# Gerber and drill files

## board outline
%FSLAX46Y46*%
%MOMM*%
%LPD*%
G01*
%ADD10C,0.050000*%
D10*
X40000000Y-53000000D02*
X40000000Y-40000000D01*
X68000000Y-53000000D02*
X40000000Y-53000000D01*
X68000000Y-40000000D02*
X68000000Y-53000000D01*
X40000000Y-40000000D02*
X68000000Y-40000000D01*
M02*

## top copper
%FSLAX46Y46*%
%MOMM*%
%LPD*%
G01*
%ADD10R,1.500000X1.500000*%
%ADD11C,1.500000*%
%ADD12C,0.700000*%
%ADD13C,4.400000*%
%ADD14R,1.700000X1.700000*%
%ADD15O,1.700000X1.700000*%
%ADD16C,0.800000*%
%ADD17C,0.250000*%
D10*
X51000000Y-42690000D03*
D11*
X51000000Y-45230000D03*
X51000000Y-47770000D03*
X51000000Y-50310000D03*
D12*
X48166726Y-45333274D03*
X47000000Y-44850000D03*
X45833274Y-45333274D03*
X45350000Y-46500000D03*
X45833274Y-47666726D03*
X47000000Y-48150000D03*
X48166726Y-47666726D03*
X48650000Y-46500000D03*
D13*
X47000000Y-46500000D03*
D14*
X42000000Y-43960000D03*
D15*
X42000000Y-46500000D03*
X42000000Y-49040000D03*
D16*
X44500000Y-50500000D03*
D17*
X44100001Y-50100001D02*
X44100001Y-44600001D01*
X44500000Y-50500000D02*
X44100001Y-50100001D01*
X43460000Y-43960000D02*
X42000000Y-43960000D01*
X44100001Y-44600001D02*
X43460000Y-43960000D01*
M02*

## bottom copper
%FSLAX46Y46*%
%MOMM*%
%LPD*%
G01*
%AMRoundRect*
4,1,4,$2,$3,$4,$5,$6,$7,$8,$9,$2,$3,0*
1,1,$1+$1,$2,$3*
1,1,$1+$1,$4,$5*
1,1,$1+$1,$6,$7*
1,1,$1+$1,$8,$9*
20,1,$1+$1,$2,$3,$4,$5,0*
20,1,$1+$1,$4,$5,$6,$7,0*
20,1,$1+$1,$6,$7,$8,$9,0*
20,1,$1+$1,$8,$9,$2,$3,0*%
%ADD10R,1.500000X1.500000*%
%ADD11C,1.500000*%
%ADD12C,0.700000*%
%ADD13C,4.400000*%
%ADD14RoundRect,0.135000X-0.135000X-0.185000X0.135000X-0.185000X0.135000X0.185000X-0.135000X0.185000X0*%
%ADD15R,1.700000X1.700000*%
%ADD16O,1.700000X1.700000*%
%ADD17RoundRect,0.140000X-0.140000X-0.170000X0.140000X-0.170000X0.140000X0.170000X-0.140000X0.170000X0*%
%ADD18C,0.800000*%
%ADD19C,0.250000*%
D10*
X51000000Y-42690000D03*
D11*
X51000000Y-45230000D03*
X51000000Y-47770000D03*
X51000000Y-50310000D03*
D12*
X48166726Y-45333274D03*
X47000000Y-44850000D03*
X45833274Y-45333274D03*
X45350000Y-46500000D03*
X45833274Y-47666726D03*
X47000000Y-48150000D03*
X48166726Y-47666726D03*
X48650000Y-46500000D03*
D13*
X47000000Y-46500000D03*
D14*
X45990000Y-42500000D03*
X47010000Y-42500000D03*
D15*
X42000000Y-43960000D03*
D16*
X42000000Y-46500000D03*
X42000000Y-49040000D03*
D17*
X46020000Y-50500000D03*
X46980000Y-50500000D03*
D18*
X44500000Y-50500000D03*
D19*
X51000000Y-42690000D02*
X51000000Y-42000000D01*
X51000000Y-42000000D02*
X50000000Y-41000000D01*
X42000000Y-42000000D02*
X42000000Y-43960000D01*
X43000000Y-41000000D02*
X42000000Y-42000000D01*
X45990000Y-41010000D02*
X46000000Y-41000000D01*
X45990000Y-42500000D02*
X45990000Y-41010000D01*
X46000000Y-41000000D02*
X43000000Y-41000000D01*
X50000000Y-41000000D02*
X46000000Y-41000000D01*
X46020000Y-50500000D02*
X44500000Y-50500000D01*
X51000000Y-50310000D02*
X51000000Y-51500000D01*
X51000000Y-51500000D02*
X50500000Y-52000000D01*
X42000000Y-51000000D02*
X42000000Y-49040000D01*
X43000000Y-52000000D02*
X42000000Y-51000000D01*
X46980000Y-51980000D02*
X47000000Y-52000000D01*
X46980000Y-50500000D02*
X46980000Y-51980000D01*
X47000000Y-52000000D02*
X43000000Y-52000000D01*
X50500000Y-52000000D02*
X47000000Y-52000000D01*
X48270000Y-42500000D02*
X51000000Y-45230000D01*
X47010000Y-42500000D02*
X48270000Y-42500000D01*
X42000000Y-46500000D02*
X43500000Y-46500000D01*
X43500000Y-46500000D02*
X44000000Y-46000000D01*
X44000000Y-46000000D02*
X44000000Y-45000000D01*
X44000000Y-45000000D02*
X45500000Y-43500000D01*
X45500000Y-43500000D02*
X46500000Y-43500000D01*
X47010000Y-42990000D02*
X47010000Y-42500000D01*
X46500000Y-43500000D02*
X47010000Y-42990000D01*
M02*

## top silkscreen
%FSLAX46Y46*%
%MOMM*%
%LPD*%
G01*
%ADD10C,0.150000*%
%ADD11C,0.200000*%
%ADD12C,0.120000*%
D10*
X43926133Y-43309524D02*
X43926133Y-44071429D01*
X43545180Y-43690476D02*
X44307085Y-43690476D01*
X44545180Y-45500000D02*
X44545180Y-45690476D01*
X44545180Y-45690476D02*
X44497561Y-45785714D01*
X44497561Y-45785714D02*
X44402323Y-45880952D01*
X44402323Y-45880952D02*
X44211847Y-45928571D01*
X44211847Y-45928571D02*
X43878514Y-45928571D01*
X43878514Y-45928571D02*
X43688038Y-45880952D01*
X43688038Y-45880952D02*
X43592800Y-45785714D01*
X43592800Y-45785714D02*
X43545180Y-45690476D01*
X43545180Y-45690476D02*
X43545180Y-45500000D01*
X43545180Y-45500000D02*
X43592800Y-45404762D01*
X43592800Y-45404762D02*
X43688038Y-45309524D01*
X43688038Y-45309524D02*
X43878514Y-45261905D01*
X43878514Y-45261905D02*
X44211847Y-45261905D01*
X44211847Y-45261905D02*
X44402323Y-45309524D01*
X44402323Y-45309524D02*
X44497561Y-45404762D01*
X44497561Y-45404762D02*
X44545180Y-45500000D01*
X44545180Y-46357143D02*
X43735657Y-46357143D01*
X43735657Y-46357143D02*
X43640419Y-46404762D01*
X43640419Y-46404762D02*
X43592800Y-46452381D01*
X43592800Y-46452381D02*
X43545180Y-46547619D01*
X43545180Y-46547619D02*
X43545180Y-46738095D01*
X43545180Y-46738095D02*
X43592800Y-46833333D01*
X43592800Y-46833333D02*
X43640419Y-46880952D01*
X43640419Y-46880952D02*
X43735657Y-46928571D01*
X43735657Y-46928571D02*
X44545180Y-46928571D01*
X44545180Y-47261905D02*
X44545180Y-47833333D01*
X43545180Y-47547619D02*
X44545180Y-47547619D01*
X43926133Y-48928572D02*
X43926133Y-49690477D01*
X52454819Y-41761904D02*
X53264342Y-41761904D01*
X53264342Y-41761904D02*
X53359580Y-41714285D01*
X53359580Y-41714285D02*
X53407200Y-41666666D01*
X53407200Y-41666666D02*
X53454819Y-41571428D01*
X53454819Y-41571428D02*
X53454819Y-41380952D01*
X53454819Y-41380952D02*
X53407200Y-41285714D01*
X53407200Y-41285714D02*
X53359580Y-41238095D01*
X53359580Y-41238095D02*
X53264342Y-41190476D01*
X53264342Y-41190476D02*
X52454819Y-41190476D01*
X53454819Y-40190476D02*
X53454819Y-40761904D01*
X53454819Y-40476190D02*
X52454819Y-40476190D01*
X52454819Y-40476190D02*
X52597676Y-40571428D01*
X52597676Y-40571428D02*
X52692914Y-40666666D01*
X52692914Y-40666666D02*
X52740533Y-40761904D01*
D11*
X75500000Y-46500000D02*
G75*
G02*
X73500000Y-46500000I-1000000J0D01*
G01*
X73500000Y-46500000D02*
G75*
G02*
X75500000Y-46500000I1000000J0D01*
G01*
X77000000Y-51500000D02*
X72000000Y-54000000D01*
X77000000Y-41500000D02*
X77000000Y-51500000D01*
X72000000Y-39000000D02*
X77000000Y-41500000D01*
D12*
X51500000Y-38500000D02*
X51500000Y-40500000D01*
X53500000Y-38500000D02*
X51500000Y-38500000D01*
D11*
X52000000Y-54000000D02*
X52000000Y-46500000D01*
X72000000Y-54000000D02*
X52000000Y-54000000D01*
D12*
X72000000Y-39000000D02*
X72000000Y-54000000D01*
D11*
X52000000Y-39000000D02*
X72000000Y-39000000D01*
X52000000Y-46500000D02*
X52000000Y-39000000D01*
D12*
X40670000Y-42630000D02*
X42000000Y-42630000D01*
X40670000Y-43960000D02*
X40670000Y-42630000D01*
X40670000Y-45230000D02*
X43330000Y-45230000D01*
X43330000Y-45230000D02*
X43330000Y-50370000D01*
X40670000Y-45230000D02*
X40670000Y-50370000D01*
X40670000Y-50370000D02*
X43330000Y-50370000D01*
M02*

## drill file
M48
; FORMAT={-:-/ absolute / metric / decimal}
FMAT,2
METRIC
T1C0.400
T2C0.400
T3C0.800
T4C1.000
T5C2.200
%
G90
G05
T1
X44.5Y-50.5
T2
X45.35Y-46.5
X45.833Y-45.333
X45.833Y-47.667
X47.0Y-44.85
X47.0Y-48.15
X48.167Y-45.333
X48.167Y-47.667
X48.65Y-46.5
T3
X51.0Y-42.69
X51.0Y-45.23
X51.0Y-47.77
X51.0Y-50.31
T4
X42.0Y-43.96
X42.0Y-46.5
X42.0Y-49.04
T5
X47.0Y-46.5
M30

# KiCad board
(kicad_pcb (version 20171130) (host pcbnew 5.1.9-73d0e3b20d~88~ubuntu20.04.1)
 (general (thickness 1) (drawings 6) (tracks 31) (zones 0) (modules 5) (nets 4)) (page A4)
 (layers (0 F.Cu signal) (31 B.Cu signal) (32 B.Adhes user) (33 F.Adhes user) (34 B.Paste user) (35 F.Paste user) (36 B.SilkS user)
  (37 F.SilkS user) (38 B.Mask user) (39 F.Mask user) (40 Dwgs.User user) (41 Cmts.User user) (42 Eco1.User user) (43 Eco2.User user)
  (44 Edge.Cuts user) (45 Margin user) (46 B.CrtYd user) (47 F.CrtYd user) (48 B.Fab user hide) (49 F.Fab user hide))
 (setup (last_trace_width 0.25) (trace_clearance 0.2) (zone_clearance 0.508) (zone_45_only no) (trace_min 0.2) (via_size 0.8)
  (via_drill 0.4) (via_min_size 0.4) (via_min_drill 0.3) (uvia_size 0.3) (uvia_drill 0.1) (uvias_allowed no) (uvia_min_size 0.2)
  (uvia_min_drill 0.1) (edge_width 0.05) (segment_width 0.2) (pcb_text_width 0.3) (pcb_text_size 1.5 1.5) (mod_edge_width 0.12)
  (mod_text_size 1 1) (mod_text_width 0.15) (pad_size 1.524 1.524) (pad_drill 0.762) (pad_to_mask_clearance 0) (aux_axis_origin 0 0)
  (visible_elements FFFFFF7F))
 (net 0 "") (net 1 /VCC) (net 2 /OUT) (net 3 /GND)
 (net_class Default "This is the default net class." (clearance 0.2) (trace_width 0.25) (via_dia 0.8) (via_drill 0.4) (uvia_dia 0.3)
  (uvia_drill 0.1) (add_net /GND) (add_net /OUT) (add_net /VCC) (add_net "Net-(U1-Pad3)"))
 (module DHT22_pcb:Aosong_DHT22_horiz (layer F.Cu) (at 51 46.5)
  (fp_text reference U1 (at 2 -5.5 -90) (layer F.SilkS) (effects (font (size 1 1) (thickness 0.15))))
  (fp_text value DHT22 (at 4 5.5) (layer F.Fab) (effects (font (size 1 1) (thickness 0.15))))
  (fp_circle (center 23.5 0) (end 24.5 0) (layer F.SilkS) (width 0.2))
  (fp_line (start 26 5) (end 21 7.5) (layer F.SilkS) (width 0.2))
  (fp_line (start 26 -5) (end 26 5) (layer F.SilkS) (width 0.2))
  (fp_line (start 21 -7.5) (end 26 -5) (layer F.SilkS) (width 0.2))
  (fp_line (start 0.5 -8) (end 0.5 -6) (layer F.SilkS) (width 0.12))
  (fp_line (start 2.5 -8) (end 0.5 -8) (layer F.SilkS) (width 0.12))
  (fp_line (start 1 7.5) (end 1 0) (layer F.SilkS) (width 0.2))
  (fp_line (start 21 7.5) (end 1 7.5) (layer F.SilkS) (width 0.2))
  (fp_line (start 21 -7.5) (end 21 7.5) (layer F.SilkS) (width 0.12))
  (fp_line (start 1 -7.5) (end 21 -7.5) (layer F.SilkS) (width 0.2))
  (fp_line (start 1 0) (end 1 -7.5) (layer F.SilkS) (width 0.2))
  (pad 1 thru_hole rect (at 0 -3.81) (size 1.5 1.5) (drill 0.8) (layers *.Cu *.Mask) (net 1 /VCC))
  (pad 2 thru_hole circle (at 0 -1.27) (size 1.5 1.5) (drill 0.8) (layers *.Cu *.Mask) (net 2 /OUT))
  (pad 3 thru_hole circle (at 0 1.27) (size 1.5 1.5) (drill 0.8) (layers *.Cu *.Mask))
  (pad 4 thru_hole circle (at 0 3.81) (size 1.5 1.5) (drill 0.8) (layers *.Cu *.Mask) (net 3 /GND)))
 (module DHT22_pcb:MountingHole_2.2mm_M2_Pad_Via (layer F.Cu) (at 47 46.5)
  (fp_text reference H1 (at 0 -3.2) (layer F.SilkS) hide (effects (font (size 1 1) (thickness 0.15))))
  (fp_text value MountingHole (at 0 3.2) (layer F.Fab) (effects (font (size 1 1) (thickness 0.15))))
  (pad 1 thru_hole circle (at 1.166726 -1.166726) (size 0.7 0.7) (drill 0.4) (layers *.Cu *.Mask))
  (pad 1 thru_hole circle (at 0 -1.65) (size 0.7 0.7) (drill 0.4) (layers *.Cu *.Mask))
  (pad 1 thru_hole circle (at -1.166726 -1.166726) (size 0.7 0.7) (drill 0.4) (layers *.Cu *.Mask))
  (pad 1 thru_hole circle (at -1.65 0) (size 0.7 0.7) (drill 0.4) (layers *.Cu *.Mask))
  (pad 1 thru_hole circle (at -1.166726 1.166726) (size 0.7 0.7) (drill 0.4) (layers *.Cu *.Mask))
  (pad 1 thru_hole circle (at 0 1.65) (size 0.7 0.7) (drill 0.4) (layers *.Cu *.Mask))
  (pad 1 thru_hole circle (at 1.166726 1.166726) (size 0.7 0.7) (drill 0.4) (layers *.Cu *.Mask))
  (pad 1 thru_hole circle (at 1.65 0) (size 0.7 0.7) (drill 0.4) (layers *.Cu *.Mask))
  (pad 1 thru_hole circle (at 0 0) (size 4.4 4.4) (drill 2.2) (layers *.Cu *.Mask)))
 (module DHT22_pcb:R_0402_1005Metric (layer B.Cu) (at 46.5 42.5)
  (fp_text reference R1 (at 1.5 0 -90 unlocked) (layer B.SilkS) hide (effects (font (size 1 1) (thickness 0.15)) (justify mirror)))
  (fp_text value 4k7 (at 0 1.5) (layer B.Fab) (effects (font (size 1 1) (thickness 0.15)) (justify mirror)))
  (pad 1 smd roundrect (at -0.51 0) (size 0.54 0.64) (layers B.Cu B.Paste B.Mask) (roundrect_rratio 0.25) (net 1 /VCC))
  (pad 2 smd roundrect (at 0.51 0) (size 0.54 0.64) (layers B.Cu B.Paste B.Mask) (roundrect_rratio 0.25) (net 2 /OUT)))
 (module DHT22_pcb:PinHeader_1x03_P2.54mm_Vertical (layer F.Cu) (at 42 43.96)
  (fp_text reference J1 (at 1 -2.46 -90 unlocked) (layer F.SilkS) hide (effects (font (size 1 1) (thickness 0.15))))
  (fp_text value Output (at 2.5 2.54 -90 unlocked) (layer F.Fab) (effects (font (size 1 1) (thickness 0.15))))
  (fp_line (start -1.33 -1.33) (end 0 -1.33) (layer F.SilkS) (width 0.12))
  (fp_line (start -1.33 0) (end -1.33 -1.33) (layer F.SilkS) (width 0.12))
  (fp_line (start -1.33 1.27) (end 1.33 1.27) (layer F.SilkS) (width 0.12))
  (fp_line (start 1.33 1.27) (end 1.33 6.41) (layer F.SilkS) (width 0.12))
  (fp_line (start -1.33 1.27) (end -1.33 6.41) (layer F.SilkS) (width 0.12))
  (fp_line (start -1.33 6.41) (end 1.33 6.41) (layer F.SilkS) (width 0.12))
  (pad 1 thru_hole rect (at 0 0) (size 1.7 1.7) (drill 1) (layers *.Cu *.Mask) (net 1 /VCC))
  (pad 2 thru_hole oval (at 0 2.54) (size 1.7 1.7) (drill 1) (layers *.Cu *.Mask) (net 2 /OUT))
  (pad 3 thru_hole oval (at 0 5.08) (size 1.7 1.7) (drill 1) (layers *.Cu *.Mask) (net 3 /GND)))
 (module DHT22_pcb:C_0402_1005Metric (layer B.Cu) (at 46.5 50.5)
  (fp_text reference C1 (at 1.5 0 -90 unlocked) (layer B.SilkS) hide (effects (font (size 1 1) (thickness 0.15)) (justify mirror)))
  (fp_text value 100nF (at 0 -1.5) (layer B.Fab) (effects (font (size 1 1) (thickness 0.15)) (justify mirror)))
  (pad 1 smd roundrect (at -0.48 0) (size 0.56 0.62) (layers B.Cu B.Paste B.Mask) (roundrect_rratio 0.25) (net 1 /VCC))
  (pad 2 smd roundrect (at 0.48 0) (size 0.56 0.62) (layers B.Cu B.Paste B.Mask) (roundrect_rratio 0.25) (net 3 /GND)))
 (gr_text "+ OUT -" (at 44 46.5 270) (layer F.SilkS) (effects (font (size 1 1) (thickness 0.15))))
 (gr_line (start 40 53) (end 40 40) (layer Edge.Cuts) (width 0.05))
 (gr_line (start 68 53) (end 40 53) (layer Edge.Cuts) (width 0.05))
 (gr_line (start 68 40) (end 68 53) (layer Edge.Cuts) (width 0.05))
 (gr_line (start 40 40) (end 68 40) (layer Edge.Cuts) (width 0.05))
 (segment (start 51 42.69) (end 51 42) (width 0.25) (layer B.Cu) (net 1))
 (segment (start 51 42) (end 50 41) (width 0.25) (layer B.Cu) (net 1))
 (segment (start 42 42) (end 42 43.96) (width 0.25) (layer B.Cu) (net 1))
 (segment (start 43 41) (end 42 42) (width 0.25) (layer B.Cu) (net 1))
 (segment (start 45.99 41.01) (end 46 41) (width 0.25) (layer B.Cu) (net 1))
 (segment (start 45.99 42.5) (end 45.99 41.01) (width 0.25) (layer B.Cu) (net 1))
 (segment (start 46 41) (end 43 41) (width 0.25) (layer B.Cu) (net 1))
 (segment (start 50 41) (end 46 41) (width 0.25) (layer B.Cu) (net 1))
 (via (at 44.5 50.5) (size 0.8) (drill 0.4) (layers F.Cu B.Cu) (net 1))
 (segment (start 46.02 50.5) (end 44.5 50.5) (width 0.25) (layer B.Cu) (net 1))
 (segment (start 44.100001 50.100001) (end 44.100001 44.600001) (width 0.25) (layer F.Cu) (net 1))
 (segment (start 44.5 50.5) (end 44.100001 50.100001) (width 0.25) (layer F.Cu) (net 1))
 (segment (start 43.46 43.96) (end 42 43.96) (width 0.25) (layer F.Cu) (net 1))
 (segment (start 44.100001 44.600001) (end 43.46 43.96) (width 0.25) (layer F.Cu) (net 1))
 (segment (start 51 50.31) (end 51 51.5) (width 0.25) (layer B.Cu) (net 3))
 (segment (start 51 51.5) (end 50.5 52) (width 0.25) (layer B.Cu) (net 3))
 (segment (start 42 51) (end 42 49.04) (width 0.25) (layer B.Cu) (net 3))
 (segment (start 43 52) (end 42 51) (width 0.25) (layer B.Cu) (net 3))
 (segment (start 46.98 51.98) (end 47 52) (width 0.25) (layer B.Cu) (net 3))
 (segment (start 46.98 50.5) (end 46.98 51.98) (width 0.25) (layer B.Cu) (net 3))
 (segment (start 47 52) (end 43 52) (width 0.25) (layer B.Cu) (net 3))
 (segment (start 50.5 52) (end 47 52) (width 0.25) (layer B.Cu) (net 3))
 (segment (start 48.27 42.5) (end 51 45.23) (width 0.25) (layer B.Cu) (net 2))
 (segment (start 47.01 42.5) (end 48.27 42.5) (width 0.25) (layer B.Cu) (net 2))
 (segment (start 42 46.5) (end 43.5 46.5) (width 0.25) (layer B.Cu) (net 2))
 (segment (start 43.5 46.5) (end 44 46) (width 0.25) (layer B.Cu) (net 2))
 (segment (start 44 46) (end 44 45) (width 0.25) (layer B.Cu) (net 2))
 (segment (start 44 45) (end 45.5 43.5) (width 0.25) (layer B.Cu) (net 2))
 (segment (start 45.5 43.5) (end 46.5 43.5) (width 0.25) (layer B.Cu) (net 2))
 (segment (start 47.01 42.99) (end 47.01 42.5) (width 0.25) (layer B.Cu) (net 2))
 (segment (start 46.5 43.5) (end 47.01 42.99) (width 0.25) (layer B.Cu) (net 2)))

